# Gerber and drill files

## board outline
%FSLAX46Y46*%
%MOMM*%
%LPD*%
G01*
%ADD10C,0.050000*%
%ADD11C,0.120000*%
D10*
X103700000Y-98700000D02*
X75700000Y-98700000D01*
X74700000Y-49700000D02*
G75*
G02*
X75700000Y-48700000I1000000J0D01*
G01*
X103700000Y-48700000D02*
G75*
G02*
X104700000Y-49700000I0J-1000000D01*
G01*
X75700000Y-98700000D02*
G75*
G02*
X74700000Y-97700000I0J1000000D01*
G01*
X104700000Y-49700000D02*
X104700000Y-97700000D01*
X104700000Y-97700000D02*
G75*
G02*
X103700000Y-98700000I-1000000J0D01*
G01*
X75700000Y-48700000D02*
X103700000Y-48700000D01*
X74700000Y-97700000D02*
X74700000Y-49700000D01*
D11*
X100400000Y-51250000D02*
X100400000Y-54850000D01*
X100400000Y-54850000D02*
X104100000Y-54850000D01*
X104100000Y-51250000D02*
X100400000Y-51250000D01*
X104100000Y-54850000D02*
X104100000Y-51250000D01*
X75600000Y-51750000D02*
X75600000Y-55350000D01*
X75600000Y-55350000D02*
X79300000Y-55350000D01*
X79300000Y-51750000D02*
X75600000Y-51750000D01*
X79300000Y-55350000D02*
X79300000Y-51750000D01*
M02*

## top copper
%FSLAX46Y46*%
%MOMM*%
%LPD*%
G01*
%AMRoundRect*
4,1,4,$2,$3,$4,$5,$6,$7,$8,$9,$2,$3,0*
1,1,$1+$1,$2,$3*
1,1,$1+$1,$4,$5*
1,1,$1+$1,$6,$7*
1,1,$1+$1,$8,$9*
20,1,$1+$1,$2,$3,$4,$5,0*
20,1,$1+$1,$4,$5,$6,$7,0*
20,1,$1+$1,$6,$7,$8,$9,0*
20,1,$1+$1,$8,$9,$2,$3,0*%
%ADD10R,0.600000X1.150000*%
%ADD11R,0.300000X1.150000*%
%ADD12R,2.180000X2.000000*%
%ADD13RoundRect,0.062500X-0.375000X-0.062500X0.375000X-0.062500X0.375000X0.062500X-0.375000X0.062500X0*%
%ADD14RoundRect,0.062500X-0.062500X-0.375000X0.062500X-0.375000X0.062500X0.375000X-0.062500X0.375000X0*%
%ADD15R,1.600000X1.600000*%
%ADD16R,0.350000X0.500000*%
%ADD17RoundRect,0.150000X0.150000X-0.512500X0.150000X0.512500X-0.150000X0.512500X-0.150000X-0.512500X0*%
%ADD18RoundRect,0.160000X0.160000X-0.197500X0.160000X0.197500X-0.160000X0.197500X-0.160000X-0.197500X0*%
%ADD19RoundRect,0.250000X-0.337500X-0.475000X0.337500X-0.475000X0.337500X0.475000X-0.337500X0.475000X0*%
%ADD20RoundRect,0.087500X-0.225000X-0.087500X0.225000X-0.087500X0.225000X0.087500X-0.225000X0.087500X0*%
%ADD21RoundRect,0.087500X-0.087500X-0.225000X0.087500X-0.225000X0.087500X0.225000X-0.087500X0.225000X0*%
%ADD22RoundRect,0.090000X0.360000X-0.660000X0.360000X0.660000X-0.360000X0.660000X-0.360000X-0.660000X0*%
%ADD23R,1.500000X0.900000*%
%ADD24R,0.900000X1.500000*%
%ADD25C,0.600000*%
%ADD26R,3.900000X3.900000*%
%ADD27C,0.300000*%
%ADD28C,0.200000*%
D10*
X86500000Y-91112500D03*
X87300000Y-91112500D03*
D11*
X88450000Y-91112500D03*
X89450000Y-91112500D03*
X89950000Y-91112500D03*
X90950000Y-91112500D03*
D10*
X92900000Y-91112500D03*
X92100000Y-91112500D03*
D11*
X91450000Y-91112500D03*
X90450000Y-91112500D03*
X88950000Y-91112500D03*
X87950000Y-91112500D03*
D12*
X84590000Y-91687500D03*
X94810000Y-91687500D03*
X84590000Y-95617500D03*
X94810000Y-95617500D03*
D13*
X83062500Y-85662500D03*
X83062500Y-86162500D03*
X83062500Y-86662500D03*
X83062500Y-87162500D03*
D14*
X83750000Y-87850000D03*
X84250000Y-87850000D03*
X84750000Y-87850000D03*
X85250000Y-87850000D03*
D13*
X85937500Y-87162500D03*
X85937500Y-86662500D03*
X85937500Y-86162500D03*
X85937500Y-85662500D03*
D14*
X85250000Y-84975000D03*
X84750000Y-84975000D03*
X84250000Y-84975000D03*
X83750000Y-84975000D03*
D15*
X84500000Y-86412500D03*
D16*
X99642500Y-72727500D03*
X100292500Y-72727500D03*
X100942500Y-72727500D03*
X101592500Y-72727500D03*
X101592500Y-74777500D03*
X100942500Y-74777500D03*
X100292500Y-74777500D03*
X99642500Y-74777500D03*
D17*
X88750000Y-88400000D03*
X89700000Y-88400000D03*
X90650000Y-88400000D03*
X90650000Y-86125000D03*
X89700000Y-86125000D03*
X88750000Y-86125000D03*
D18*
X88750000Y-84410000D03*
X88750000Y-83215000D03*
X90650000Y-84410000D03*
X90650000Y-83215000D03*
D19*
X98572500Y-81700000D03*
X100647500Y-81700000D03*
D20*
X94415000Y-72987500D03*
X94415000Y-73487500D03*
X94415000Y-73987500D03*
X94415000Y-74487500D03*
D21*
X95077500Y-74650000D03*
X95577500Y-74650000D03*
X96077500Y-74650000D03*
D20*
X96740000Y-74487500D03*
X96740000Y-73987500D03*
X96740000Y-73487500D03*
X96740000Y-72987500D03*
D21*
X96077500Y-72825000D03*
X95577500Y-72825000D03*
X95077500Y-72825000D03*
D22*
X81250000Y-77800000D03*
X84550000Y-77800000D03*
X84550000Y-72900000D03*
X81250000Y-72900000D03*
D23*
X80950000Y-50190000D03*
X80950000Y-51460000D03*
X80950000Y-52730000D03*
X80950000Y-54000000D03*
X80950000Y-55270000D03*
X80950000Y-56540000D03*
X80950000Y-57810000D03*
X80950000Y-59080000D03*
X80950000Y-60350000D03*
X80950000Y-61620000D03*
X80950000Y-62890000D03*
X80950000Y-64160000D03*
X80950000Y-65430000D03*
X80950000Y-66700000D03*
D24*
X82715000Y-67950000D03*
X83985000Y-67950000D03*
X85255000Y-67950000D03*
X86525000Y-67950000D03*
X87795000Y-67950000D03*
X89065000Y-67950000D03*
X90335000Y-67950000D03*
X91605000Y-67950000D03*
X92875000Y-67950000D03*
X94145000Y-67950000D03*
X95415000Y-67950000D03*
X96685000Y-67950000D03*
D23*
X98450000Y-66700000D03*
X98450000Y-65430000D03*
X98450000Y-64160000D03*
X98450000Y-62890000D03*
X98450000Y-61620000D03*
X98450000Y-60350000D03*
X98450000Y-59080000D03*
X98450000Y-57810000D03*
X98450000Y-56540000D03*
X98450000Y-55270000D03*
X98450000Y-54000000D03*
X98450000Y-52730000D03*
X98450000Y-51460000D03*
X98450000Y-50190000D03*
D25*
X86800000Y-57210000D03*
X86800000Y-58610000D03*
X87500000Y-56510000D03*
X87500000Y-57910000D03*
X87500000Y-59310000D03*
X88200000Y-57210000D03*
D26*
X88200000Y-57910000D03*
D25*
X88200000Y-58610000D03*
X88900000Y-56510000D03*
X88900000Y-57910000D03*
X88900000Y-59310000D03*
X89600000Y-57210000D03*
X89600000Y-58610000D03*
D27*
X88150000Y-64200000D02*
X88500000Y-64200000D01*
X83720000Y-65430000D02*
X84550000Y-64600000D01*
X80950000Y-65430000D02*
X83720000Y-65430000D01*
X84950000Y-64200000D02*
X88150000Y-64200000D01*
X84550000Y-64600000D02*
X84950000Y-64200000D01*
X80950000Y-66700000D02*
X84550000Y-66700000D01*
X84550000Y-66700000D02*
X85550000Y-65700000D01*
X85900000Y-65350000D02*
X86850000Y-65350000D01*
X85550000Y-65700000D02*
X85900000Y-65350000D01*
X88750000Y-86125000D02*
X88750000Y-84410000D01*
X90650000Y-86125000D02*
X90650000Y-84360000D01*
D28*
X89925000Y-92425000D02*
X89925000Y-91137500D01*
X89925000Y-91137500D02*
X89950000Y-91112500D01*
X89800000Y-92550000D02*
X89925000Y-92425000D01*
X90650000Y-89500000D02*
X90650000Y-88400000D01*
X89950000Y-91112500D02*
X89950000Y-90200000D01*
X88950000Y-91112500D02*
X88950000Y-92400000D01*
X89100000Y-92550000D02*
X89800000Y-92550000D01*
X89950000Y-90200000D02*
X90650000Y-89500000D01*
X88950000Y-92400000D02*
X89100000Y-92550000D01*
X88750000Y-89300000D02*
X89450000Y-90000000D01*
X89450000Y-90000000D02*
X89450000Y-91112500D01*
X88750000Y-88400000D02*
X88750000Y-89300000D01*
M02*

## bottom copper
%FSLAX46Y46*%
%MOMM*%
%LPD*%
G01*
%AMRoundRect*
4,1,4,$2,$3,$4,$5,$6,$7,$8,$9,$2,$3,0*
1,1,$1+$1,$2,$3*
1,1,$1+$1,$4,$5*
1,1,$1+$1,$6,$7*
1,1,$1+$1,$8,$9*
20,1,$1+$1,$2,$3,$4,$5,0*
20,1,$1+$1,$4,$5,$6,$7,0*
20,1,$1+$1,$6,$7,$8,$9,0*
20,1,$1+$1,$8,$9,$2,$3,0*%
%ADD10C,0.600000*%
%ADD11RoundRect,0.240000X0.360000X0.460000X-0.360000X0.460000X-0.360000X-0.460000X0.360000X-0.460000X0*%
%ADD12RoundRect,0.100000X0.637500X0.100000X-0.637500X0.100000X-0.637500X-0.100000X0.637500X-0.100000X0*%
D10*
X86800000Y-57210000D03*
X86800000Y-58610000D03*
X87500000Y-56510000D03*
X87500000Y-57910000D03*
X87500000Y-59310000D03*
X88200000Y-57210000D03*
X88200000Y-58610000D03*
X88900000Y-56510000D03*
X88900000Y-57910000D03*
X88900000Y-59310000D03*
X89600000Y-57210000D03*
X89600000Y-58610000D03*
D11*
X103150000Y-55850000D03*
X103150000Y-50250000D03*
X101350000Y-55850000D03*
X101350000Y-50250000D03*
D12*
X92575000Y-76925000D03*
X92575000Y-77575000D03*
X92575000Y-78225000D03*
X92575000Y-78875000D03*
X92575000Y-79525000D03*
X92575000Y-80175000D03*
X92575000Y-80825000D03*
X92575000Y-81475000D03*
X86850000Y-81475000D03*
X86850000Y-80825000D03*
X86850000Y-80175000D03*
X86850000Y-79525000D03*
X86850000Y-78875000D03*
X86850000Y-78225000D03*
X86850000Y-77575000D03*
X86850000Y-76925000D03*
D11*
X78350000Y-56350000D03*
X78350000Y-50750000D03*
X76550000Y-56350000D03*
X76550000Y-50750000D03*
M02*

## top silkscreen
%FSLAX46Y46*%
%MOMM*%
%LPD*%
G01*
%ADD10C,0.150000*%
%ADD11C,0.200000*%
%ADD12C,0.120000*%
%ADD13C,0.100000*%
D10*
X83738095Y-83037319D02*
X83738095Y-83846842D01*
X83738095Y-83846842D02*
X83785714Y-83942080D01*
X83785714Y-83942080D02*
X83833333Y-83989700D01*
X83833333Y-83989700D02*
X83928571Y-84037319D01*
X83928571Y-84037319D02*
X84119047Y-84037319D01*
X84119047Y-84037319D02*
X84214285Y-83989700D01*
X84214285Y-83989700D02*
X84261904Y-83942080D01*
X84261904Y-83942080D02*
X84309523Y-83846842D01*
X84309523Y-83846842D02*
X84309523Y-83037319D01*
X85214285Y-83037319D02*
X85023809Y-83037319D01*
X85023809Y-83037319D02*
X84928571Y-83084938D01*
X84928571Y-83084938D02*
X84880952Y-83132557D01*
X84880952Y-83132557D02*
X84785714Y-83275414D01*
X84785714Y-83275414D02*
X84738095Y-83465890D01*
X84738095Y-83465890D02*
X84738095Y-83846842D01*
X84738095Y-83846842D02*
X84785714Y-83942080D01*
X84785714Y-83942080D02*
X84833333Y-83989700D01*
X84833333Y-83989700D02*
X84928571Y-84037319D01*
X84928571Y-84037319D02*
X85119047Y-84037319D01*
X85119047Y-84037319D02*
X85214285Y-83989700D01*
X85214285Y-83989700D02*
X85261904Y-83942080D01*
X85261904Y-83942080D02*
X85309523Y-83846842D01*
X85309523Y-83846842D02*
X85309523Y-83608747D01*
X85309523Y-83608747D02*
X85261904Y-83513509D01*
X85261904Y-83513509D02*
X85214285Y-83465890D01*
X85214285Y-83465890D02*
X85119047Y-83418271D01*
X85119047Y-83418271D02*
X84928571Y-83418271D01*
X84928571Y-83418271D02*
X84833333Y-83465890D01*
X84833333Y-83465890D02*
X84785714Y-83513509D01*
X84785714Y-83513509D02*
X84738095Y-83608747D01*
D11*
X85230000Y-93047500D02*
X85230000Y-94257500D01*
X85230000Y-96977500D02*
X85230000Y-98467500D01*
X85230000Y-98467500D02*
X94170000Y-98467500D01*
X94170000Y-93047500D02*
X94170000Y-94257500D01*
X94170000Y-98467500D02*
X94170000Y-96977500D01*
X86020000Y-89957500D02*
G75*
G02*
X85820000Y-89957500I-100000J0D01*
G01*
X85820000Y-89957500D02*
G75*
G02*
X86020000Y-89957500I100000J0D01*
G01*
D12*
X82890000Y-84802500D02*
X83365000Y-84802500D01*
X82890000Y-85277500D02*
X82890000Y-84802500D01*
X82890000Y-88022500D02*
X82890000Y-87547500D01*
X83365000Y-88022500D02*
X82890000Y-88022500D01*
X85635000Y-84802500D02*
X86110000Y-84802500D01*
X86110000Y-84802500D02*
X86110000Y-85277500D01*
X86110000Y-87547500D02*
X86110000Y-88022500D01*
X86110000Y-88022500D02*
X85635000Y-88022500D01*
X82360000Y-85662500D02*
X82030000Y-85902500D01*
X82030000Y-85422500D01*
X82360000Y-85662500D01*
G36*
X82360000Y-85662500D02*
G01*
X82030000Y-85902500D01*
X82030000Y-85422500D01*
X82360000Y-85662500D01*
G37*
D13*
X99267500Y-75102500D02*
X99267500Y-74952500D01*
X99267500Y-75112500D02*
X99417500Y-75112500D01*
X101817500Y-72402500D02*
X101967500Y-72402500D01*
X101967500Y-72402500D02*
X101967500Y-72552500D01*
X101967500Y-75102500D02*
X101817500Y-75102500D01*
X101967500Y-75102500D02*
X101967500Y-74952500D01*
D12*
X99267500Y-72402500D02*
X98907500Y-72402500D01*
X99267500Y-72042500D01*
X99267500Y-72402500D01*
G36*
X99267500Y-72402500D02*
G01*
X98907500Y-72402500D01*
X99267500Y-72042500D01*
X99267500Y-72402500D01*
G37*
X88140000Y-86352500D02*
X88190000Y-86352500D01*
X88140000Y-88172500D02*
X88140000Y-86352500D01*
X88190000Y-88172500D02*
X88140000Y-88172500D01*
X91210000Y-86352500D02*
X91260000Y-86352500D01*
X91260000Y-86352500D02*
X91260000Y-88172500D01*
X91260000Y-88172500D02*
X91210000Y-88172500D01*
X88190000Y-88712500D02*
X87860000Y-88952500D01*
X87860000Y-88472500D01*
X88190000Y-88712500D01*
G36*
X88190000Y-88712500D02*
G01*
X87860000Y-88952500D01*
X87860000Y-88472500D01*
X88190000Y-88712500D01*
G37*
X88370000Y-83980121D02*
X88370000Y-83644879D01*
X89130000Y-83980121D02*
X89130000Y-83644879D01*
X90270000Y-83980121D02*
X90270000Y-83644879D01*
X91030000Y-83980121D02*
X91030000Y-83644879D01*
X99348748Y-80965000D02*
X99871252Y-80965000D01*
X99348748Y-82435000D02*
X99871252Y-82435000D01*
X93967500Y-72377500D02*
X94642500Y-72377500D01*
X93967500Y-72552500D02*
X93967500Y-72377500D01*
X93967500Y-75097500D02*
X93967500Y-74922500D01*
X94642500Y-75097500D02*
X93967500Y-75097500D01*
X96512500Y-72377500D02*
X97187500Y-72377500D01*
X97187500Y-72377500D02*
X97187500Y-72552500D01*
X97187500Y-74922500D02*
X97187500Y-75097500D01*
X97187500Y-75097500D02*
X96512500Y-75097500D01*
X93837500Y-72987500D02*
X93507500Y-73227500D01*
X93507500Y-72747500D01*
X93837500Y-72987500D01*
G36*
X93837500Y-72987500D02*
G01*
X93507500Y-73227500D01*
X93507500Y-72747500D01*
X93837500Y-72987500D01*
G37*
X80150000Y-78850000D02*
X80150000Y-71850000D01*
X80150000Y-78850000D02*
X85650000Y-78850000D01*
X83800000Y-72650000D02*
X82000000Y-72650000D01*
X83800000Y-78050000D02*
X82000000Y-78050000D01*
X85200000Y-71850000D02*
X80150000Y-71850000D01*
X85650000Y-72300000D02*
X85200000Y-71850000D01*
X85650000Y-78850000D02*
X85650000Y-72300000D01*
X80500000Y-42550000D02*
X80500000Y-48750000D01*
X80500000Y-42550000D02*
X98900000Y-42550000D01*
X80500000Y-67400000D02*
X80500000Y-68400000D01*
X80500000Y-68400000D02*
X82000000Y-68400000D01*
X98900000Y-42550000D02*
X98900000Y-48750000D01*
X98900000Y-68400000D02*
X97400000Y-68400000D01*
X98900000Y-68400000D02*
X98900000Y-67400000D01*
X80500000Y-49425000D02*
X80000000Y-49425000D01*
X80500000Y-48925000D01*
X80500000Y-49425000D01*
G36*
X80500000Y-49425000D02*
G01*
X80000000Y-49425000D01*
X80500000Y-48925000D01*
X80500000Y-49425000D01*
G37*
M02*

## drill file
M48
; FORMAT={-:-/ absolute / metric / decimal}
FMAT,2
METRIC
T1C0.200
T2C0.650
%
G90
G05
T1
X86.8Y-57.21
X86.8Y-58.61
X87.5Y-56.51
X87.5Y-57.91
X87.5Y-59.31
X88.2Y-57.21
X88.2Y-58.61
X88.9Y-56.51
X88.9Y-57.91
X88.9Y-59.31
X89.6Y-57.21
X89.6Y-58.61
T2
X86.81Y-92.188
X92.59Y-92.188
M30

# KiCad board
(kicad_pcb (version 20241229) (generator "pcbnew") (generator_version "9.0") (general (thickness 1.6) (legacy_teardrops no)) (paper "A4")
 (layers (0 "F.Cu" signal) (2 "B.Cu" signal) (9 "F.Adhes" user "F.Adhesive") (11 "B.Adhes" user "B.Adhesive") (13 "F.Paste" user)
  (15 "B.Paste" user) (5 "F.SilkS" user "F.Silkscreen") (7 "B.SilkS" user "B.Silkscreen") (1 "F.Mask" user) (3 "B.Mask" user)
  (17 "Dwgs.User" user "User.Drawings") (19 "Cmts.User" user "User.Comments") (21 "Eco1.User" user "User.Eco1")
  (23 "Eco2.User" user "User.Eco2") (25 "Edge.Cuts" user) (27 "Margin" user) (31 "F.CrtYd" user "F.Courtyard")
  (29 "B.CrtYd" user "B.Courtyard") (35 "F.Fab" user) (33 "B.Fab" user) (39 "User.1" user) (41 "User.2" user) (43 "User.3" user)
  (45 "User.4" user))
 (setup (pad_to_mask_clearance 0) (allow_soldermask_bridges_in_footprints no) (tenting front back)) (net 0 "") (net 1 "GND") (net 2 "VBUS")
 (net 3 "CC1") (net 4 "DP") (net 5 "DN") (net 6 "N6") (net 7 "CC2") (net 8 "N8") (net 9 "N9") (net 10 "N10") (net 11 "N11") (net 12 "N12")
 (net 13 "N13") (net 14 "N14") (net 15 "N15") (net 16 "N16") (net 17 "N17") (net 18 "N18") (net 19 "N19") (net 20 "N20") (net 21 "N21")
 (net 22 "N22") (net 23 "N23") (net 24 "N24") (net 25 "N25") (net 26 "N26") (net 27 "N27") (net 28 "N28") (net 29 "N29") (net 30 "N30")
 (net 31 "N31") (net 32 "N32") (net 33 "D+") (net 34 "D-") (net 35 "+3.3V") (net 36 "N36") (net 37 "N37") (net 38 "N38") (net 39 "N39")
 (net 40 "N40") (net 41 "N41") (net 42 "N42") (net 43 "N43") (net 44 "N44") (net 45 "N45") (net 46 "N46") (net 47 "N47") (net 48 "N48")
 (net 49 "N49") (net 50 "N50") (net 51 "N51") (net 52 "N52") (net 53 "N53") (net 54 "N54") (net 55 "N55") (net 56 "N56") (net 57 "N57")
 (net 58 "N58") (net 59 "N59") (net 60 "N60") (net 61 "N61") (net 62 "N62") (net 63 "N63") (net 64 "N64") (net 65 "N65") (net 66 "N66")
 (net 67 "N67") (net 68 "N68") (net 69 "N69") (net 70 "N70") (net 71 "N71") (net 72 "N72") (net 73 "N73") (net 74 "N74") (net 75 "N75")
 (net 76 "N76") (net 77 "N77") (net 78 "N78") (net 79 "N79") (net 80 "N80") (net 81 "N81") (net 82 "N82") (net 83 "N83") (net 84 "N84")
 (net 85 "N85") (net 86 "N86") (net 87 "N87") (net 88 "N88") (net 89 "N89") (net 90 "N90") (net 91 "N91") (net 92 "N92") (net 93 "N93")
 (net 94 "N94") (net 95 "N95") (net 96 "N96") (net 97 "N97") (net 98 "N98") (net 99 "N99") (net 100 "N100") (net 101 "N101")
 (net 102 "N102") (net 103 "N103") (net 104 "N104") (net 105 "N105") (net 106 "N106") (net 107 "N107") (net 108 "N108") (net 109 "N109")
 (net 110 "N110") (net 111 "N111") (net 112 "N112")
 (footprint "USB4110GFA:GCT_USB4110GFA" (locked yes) (layer "F.Cu") (at 89.7 92.1875)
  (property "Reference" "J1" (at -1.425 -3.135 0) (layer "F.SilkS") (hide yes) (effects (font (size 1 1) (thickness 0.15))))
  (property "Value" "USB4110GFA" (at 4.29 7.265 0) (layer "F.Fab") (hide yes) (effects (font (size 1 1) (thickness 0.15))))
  (fp_line (start -4.47 0.86) (end -4.47 2.07) (stroke (width 0.2) (type solid)) (layer "F.SilkS"))
  (fp_line (start -4.47 4.79) (end -4.47 6.28) (stroke (width 0.2) (type solid)) (layer "F.SilkS"))
  (fp_line (start -4.47 6.28) (end 4.47 6.28) (stroke (width 0.2) (type solid)) (layer "F.SilkS"))
  (fp_line (start 4.47 0.86) (end 4.47 2.07) (stroke (width 0.2) (type solid)) (layer "F.SilkS"))
  (fp_line (start 4.47 6.28) (end 4.47 4.79) (stroke (width 0.2) (type solid)) (layer "F.SilkS"))
  (fp_circle (center -3.78 -2.23) (end -3.68 -2.23) (stroke (width 0.2) (type solid)) (fill no) (layer "F.SilkS"))
  (pad "" np_thru_hole circle (at -2.89 0) (size 0.65 0.65) (drill 0.65) (layers "*.Cu" "*.Mask"))
  (pad "" np_thru_hole circle (at 2.89 0) (size 0.65 0.65) (drill 0.65) (layers "*.Cu" "*.Mask"))
  (pad "A1/B12" smd rect (at -3.2 -1.075) (size 0.6 1.15) (layers "F.Cu" "F.Mask" "F.Paste") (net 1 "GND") (solder_mask_margin 0.102))
  (pad "A4/B9" smd rect (at -2.4 -1.075) (size 0.6 1.15) (layers "F.Cu" "F.Mask" "F.Paste") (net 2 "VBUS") (solder_mask_margin 0.102))
  (pad "A5" smd rect (at -1.25 -1.075) (size 0.3 1.15) (layers "F.Cu" "F.Mask" "F.Paste") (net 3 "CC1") (solder_mask_margin 0.102))
  (pad "A6" smd rect (at -0.25 -1.075) (size 0.3 1.15) (layers "F.Cu" "F.Mask" "F.Paste") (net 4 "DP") (solder_mask_margin 0.102))
  (pad "A7" smd rect (at 0.25 -1.075) (size 0.3 1.15) (layers "F.Cu" "F.Mask" "F.Paste") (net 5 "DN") (solder_mask_margin 0.102))
  (pad "A8" smd rect (at 1.25 -1.075) (size 0.3 1.15) (layers "F.Cu" "F.Mask" "F.Paste") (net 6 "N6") (solder_mask_margin 0.102))
  (pad "B1/A12" smd rect (at 3.2 -1.075) (size 0.6 1.15) (layers "F.Cu" "F.Mask" "F.Paste") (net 1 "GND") (solder_mask_margin 0.102))
  (pad "B4/A9" smd rect (at 2.4 -1.075) (size 0.6 1.15) (layers "F.Cu" "F.Mask" "F.Paste") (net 2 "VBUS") (solder_mask_margin 0.102))
  (pad "B5" smd rect (at 1.75 -1.075) (size 0.3 1.15) (layers "F.Cu" "F.Mask" "F.Paste") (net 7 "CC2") (solder_mask_margin 0.102))
  (pad "B6" smd rect (at 0.75 -1.075) (size 0.3 1.15) (layers "F.Cu" "F.Mask" "F.Paste") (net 4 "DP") (solder_mask_margin 0.102))
  (pad "B7" smd rect (at -0.75 -1.075) (size 0.3 1.15) (layers "F.Cu" "F.Mask" "F.Paste") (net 5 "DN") (solder_mask_margin 0.102))
  (pad "B8" smd rect (at -1.75 -1.075) (size 0.3 1.15) (layers "F.Cu" "F.Mask" "F.Paste") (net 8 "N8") (solder_mask_margin 0.102))
  (pad "S1" smd rect (at -5.11 -0.5) (size 2.18 2) (layers "F.Cu" "F.Mask" "F.Paste") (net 1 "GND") (solder_mask_margin 0.102))
  (pad "S2" smd rect (at 5.11 -0.5) (size 2.18 2) (layers "F.Cu" "F.Mask" "F.Paste") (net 1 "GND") (solder_mask_margin 0.102))
  (pad "S3" smd rect (at -5.11 3.43) (size 2.18 2) (layers "F.Cu" "F.Mask" "F.Paste") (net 1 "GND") (solder_mask_margin 0.102))
  (pad "S4" smd rect (at 5.11 3.43) (size 2.18 2) (layers "F.Cu" "F.Mask" "F.Paste") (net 1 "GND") (solder_mask_margin 0.102)))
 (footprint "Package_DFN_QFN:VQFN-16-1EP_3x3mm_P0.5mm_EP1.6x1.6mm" (layer "F.Cu") (at 84.5 86.4125)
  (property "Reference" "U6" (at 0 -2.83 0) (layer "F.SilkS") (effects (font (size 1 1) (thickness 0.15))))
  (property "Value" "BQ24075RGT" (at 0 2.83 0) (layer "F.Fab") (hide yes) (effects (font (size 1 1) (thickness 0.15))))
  (fp_line (start -1.61 -1.61) (end -1.135 -1.61) (stroke (width 0.12) (type solid)) (layer "F.SilkS"))
  (fp_line (start -1.61 -1.135) (end -1.61 -1.61) (stroke (width 0.12) (type solid)) (layer "F.SilkS"))
  (fp_line (start -1.61 1.61) (end -1.61 1.135) (stroke (width 0.12) (type solid)) (layer "F.SilkS"))
  (fp_line (start -1.135 1.61) (end -1.61 1.61) (stroke (width 0.12) (type solid)) (layer "F.SilkS"))
  (fp_line (start 1.135 -1.61) (end 1.61 -1.61) (stroke (width 0.12) (type solid)) (layer "F.SilkS"))
  (fp_line (start 1.61 -1.61) (end 1.61 -1.135) (stroke (width 0.12) (type solid)) (layer "F.SilkS"))
  (fp_line (start 1.61 1.135) (end 1.61 1.61) (stroke (width 0.12) (type solid)) (layer "F.SilkS"))
  (fp_line (start 1.61 1.61) (end 1.135 1.61) (stroke (width 0.12) (type solid)) (layer "F.SilkS"))
  (fp_poly (pts (xy -2.14 -0.75) (xy -2.47 -0.51) (xy -2.47 -0.99)) (stroke (width 0.12) (type solid)) (fill yes) (layer "F.SilkS"))
  (pad "" smd roundrect (at -0.4 -0.4) (size 0.64 0.64) (layers "F.Paste") (roundrect_rratio 0.25))
  (pad "" smd roundrect (at -0.4 0.4) (size 0.64 0.64) (layers "F.Paste") (roundrect_rratio 0.25))
  (pad "" smd roundrect (at 0.4 -0.4) (size 0.64 0.64) (layers "F.Paste") (roundrect_rratio 0.25))
  (pad "" smd roundrect (at 0.4 0.4) (size 0.64 0.64) (layers "F.Paste") (roundrect_rratio 0.25))
  (pad "1" smd roundrect (at -1.4375 -0.75) (size 0.875 0.25) (layers "F.Cu" "F.Mask" "F.Paste") (roundrect_rratio 0.25) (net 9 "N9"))
  (pad "2" smd roundrect (at -1.4375 -0.25) (size 0.875 0.25) (layers "F.Cu" "F.Mask" "F.Paste") (roundrect_rratio 0.25) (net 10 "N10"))
  (pad "3" smd roundrect (at -1.4375 0.25) (size 0.875 0.25) (layers "F.Cu" "F.Mask" "F.Paste") (roundrect_rratio 0.25) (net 10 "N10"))
  (pad "4" smd roundrect (at -1.4375 0.75) (size 0.875 0.25) (layers "F.Cu" "F.Mask" "F.Paste") (roundrect_rratio 0.25) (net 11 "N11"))
  (pad "5" smd roundrect (at -0.75 1.4375) (size 0.25 0.875) (layers "F.Cu" "F.Mask" "F.Paste") (roundrect_rratio 0.25) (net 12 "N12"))
  (pad "6" smd roundrect (at -0.25 1.4375) (size 0.25 0.875) (layers "F.Cu" "F.Mask" "F.Paste") (roundrect_rratio 0.25) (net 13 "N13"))
  (pad "7" smd roundrect (at 0.25 1.4375) (size 0.25 0.875) (layers "F.Cu" "F.Mask" "F.Paste") (roundrect_rratio 0.25) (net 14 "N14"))
  (pad "8" smd roundrect (at 0.75 1.4375) (size 0.25 0.875) (layers "F.Cu" "F.Mask" "F.Paste") (roundrect_rratio 0.25) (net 1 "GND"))
  (pad "9" smd roundrect (at 1.4375 0.75) (size 0.875 0.25) (layers "F.Cu" "F.Mask" "F.Paste") (roundrect_rratio 0.25) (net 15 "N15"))
  (pad "10" smd roundrect (at 1.4375 0.25) (size 0.875 0.25) (layers "F.Cu" "F.Mask" "F.Paste") (roundrect_rratio 0.25) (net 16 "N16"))
  (pad "11" smd roundrect (at 1.4375 -0.25) (size 0.875 0.25) (layers "F.Cu" "F.Mask" "F.Paste") (roundrect_rratio 0.25) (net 16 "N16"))
  (pad "12" smd roundrect (at 1.4375 -0.75) (size 0.875 0.25) (layers "F.Cu" "F.Mask" "F.Paste") (roundrect_rratio 0.25) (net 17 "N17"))
  (pad "13" smd roundrect (at 0.75 -1.4375) (size 0.25 0.875) (layers "F.Cu" "F.Mask" "F.Paste") (roundrect_rratio 0.25) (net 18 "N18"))
  (pad "14" smd roundrect (at 0.25 -1.4375) (size 0.25 0.875) (layers "F.Cu" "F.Mask" "F.Paste") (roundrect_rratio 0.25) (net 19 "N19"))
  (pad "15" smd roundrect (at -0.25 -1.4375) (size 0.25 0.875) (layers "F.Cu" "F.Mask" "F.Paste") (roundrect_rratio 0.25) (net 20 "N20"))
  (pad "16" smd roundrect (at -0.75 -1.4375) (size 0.25 0.875) (layers "F.Cu" "F.Mask" "F.Paste") (roundrect_rratio 0.25) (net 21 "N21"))
  (pad "17" smd rect (at 0 0) (size 1.6 1.6) (layers "F.Cu" "F.Mask") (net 1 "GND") (zone_connect 2)))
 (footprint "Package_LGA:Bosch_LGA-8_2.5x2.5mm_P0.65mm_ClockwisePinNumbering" (layer "F.Cu") (at 100.6175 73.7525)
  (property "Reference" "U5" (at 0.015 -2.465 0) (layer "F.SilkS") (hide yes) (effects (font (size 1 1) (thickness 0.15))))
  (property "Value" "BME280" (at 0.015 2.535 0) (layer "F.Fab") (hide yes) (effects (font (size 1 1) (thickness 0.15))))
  (fp_line (start -1.35 1.35) (end -1.35 1.2) (stroke (width 0.1) (type solid)) (layer "F.SilkS"))
  (fp_line (start -1.35 1.36) (end -1.2 1.36) (stroke (width 0.1) (type solid)) (layer "F.SilkS"))
  (fp_line (start 1.2 -1.35) (end 1.35 -1.35) (stroke (width 0.1) (type solid)) (layer "F.SilkS"))
  (fp_line (start 1.35 -1.35) (end 1.35 -1.2) (stroke (width 0.1) (type solid)) (layer "F.SilkS"))
  (fp_line (start 1.35 1.35) (end 1.2 1.35) (stroke (width 0.1) (type solid)) (layer "F.SilkS"))
  (fp_line (start 1.35 1.35) (end 1.35 1.2) (stroke (width 0.1) (type solid)) (layer "F.SilkS"))
  (fp_poly
   (pts (xy -1.35 -1.35) (xy -1.71 -1.35) (xy -1.35 -1.71) (xy -1.35 -1.35)) (stroke (width 0.12) (type solid)) (fill yes) (layer "F.SilkS"))
  (pad "1" smd rect (at -0.975 -1.025 90) (size 0.5 0.35) (layers "F.Cu" "F.Mask" "F.Paste") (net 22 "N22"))
  (pad "2" smd rect (at -0.325 -1.025 90) (size 0.5 0.35) (layers "F.Cu" "F.Mask" "F.Paste") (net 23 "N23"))
  (pad "3" smd rect (at 0.325 -1.025 90) (size 0.5 0.35) (layers "F.Cu" "F.Mask" "F.Paste") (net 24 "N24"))
  (pad "4" smd rect (at 0.975 -1.025 90) (size 0.5 0.35) (layers "F.Cu" "F.Mask" "F.Paste") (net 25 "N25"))
  (pad "5" smd rect (at 0.975 1.025 90) (size 0.5 0.35) (layers "F.Cu" "F.Mask" "F.Paste") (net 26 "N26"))
  (pad "6" smd rect (at 0.325 1.025 90) (size 0.5 0.35) (layers "F.Cu" "F.Mask" "F.Paste") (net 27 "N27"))
  (pad "7" smd rect (at -0.325 1.025 90) (size 0.5 0.35) (layers "F.Cu" "F.Mask" "F.Paste") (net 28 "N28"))
  (pad "8" smd rect (at -0.975 1.025 90) (size 0.5 0.35) (layers "F.Cu" "F.Mask" "F.Paste") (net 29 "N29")))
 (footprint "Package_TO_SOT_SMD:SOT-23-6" (layer "F.Cu") (at 89.7 87.2625 90)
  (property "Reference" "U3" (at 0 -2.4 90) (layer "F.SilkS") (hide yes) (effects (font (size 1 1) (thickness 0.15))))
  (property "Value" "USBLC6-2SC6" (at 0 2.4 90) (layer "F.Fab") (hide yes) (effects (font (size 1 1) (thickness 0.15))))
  (fp_line (start 0.91 -1.56) (end 0.91 -1.51) (stroke (width 0.12) (type solid)) (layer "F.SilkS"))
  (fp_line (start -0.91 -1.56) (end 0.91 -1.56) (stroke (width 0.12) (type solid)) (layer "F.SilkS"))
  (fp_line (start -0.91 -1.51) (end -0.91 -1.56) (stroke (width 0.12) (type solid)) (layer "F.SilkS"))
  (fp_line (start 0.91 1.51) (end 0.91 1.56) (stroke (width 0.12) (type solid)) (layer "F.SilkS"))
  (fp_line (start 0.91 1.56) (end -0.91 1.56) (stroke (width 0.12) (type solid)) (layer "F.SilkS"))
  (fp_line (start -0.91 1.56) (end -0.91 1.51) (stroke (width 0.12) (type solid)) (layer "F.SilkS"))
  (fp_poly (pts (xy -1.45 -1.51) (xy -1.69 -1.84) (xy -1.21 -1.84)) (stroke (width 0.12) (type solid)) (fill yes) (layer "F.SilkS"))
  (pad "1" smd roundrect (at -1.1375 -0.95 90) (size 1.325 0.6) (layers "F.Cu" "F.Mask" "F.Paste") (roundrect_rratio 0.25) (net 4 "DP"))
  (pad "2" smd roundrect (at -1.1375 0 90) (size 1.325 0.6) (layers "F.Cu" "F.Mask" "F.Paste") (roundrect_rratio 0.25) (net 1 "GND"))
  (pad "3" smd roundrect (at -1.1375 0.95 90) (size 1.325 0.6) (layers "F.Cu" "F.Mask" "F.Paste") (roundrect_rratio 0.25) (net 5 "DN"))
  (pad "4" smd roundrect (at 1.1375 0.95 90) (size 1.325 0.6) (layers "F.Cu" "F.Mask" "F.Paste") (roundrect_rratio 0.25) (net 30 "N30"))
  (pad "5" smd roundrect (at 1.1375 0 90) (size 1.325 0.6) (layers "F.Cu" "F.Mask" "F.Paste") (roundrect_rratio 0.25) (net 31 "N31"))
  (pad "6" smd roundrect (at 1.1375 -0.95 90) (size 1.325 0.6) (layers "F.Cu" "F.Mask" "F.Paste") (roundrect_rratio 0.25) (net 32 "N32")))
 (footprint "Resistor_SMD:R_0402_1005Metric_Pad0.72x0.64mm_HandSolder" (layer "F.Cu") (at 88.75 83.8125 90)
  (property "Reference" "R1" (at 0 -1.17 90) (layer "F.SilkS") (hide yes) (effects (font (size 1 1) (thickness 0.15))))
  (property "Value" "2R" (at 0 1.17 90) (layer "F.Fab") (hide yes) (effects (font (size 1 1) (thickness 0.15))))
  (fp_line (start -0.167621 -0.38) (end 0.167621 -0.38) (stroke (width 0.12) (type solid)) (layer "F.SilkS"))
  (fp_line (start -0.167621 0.38) (end 0.167621 0.38) (stroke (width 0.12) (type solid)) (layer "F.SilkS"))
  (pad "1" smd roundrect (at -0.5975 0 90) (size 0.715 0.64) (layers "F.Cu" "F.Mask" "F.Paste") (roundrect_rratio 0.25) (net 32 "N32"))
  (pad "2" smd roundrect (at 0.5975 0 90) (size 0.715 0.64) (layers "F.Cu" "F.Mask" "F.Paste") (roundrect_rratio 0.25) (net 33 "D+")))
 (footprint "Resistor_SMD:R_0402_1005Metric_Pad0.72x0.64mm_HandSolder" (layer "F.Cu") (at 90.65 83.8125 90)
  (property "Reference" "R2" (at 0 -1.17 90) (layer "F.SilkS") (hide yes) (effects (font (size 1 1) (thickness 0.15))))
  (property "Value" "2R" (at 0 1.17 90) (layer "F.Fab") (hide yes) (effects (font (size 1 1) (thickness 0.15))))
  (fp_line (start -0.167621 -0.38) (end 0.167621 -0.38) (stroke (width 0.12) (type solid)) (layer "F.SilkS"))
  (fp_line (start -0.167621 0.38) (end 0.167621 0.38) (stroke (width 0.12) (type solid)) (layer "F.SilkS"))
  (pad "1" smd roundrect (at -0.5975 0 90) (size 0.715 0.64) (layers "F.Cu" "F.Mask" "F.Paste") (roundrect_rratio 0.25) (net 30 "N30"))
  (pad "2" smd roundrect (at 0.5975 0 90) (size 0.715 0.64) (layers "F.Cu" "F.Mask" "F.Paste") (roundrect_rratio 0.25) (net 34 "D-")))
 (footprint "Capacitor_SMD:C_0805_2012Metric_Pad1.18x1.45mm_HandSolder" (layer "F.Cu") (at 99.61 81.7)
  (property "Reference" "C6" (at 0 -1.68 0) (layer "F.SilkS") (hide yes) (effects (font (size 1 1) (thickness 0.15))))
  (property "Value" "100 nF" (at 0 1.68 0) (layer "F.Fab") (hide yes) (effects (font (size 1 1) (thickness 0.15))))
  (fp_line (start -0.261252 -0.735) (end 0.261252 -0.735) (stroke (width 0.12) (type solid)) (layer "F.SilkS"))
  (fp_line (start -0.261252 0.735) (end 0.261252 0.735) (stroke (width 0.12) (type solid)) (layer "F.SilkS"))
  (pad "1" smd roundrect (at -1.0375 0) (size 1.175 1.45) (layers "F.Cu" "F.Mask" "F.Paste") (roundrect_rratio 0.212766) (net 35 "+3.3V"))
  (pad "2" smd roundrect (at 1.0375 0) (size 1.175 1.45) (layers "F.Cu" "F.Mask" "F.Paste") (roundrect_rratio 0.212766) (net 1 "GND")))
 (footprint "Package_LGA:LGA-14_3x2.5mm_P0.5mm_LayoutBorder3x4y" (layer "F.Cu") (at 95.5775 73.7375)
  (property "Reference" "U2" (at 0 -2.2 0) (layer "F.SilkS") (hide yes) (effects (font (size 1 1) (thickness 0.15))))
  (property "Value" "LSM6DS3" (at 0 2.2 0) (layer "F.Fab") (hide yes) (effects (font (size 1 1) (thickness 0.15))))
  (fp_line (start -1.61 -1.36) (end -0.935 -1.36) (stroke (width 0.12) (type solid)) (layer "F.SilkS"))
  (fp_line (start -1.61 -1.185) (end -1.61 -1.36) (stroke (width 0.12) (type solid)) (layer "F.SilkS"))
  (fp_line (start -1.61 1.36) (end -1.61 1.185) (stroke (width 0.12) (type solid)) (layer "F.SilkS"))
  (fp_line (start -0.935 1.36) (end -1.61 1.36) (stroke (width 0.12) (type solid)) (layer "F.SilkS"))
  (fp_line (start 0.935 -1.36) (end 1.61 -1.36) (stroke (width 0.12) (type solid)) (layer "F.SilkS"))
  (fp_line (start 1.61 -1.36) (end 1.61 -1.185) (stroke (width 0.12) (type solid)) (layer "F.SilkS"))
  (fp_line (start 1.61 1.185) (end 1.61 1.36) (stroke (width 0.12) (type solid)) (layer "F.SilkS"))
  (fp_line (start 1.61 1.36) (end 0.935 1.36) (stroke (width 0.12) (type solid)) (layer "F.SilkS"))
  (fp_poly (pts (xy -1.74 -0.75) (xy -2.07 -0.51) (xy -2.07 -0.99)) (stroke (width 0.12) (type solid)) (fill yes) (layer "F.SilkS"))
  (pad "1" smd roundrect (at -1.1625 -0.75) (size 0.625 0.35) (layers "F.Cu" "F.Mask" "F.Paste") (roundrect_rratio 0.25) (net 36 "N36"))
  (pad "2" smd roundrect (at -1.1625 -0.25) (size 0.625 0.35) (layers "F.Cu" "F.Mask" "F.Paste") (roundrect_rratio 0.25) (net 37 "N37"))
  (pad "3" smd roundrect (at -1.1625 0.25) (size 0.625 0.35) (layers "F.Cu" "F.Mask" "F.Paste") (roundrect_rratio 0.25) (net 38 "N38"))
  (pad "4" smd roundrect (at -1.1625 0.75) (size 0.625 0.35) (layers "F.Cu" "F.Mask" "F.Paste") (roundrect_rratio 0.25) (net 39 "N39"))
  (pad "5" smd roundrect (at -0.5 0.9125) (size 0.35 0.625) (layers "F.Cu" "F.Mask" "F.Paste") (roundrect_rratio 0.25) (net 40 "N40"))
  (pad "6" smd roundrect (at 0 0.9125) (size 0.35 0.625) (layers "F.Cu" "F.Mask" "F.Paste") (roundrect_rratio 0.25) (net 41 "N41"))
  (pad "7" smd roundrect (at 0.5 0.9125) (size 0.35 0.625) (layers "F.Cu" "F.Mask" "F.Paste") (roundrect_rratio 0.25) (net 41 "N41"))
  (pad "8" smd roundrect (at 1.1625 0.75) (size 0.625 0.35) (layers "F.Cu" "F.Mask" "F.Paste") (roundrect_rratio 0.25) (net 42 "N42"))
  (pad "9" smd roundrect (at 1.1625 0.25) (size 0.625 0.35) (layers "F.Cu" "F.Mask" "F.Paste") (roundrect_rratio 0.25) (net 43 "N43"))
  (pad "10" smd roundrect (at 1.1625 -0.25) (size 0.625 0.35) (layers "F.Cu" "F.Mask" "F.Paste") (roundrect_rratio 0.25) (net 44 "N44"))
  (pad "11" smd roundrect (at 1.1625 -0.75) (size 0.625 0.35) (layers "F.Cu" "F.Mask" "F.Paste") (roundrect_rratio 0.25) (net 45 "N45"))
  (pad "12" smd roundrect (at 0.5 -0.9125) (size 0.35 0.625) (layers "F.Cu" "F.Mask" "F.Paste") (roundrect_rratio 0.25) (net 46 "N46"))
  (pad "13" smd roundrect (at 0 -0.9125) (size 0.35 0.625) (layers "F.Cu" "F.Mask" "F.Paste") (roundrect_rratio 0.25) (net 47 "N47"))
  (pad "14" smd roundrect (at -0.5 -0.9125) (size 0.35 0.625) (layers "F.Cu" "F.Mask" "F.Paste") (roundrect_rratio 0.25) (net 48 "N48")))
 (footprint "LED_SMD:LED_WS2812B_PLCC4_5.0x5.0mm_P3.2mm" (layer "F.Cu") (at 82.9 75.35 90)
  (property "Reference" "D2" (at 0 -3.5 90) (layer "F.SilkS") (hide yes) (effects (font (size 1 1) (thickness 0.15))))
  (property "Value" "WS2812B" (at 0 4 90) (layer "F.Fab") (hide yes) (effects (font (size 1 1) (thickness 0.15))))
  (fp_line (start -3.5 -2.75) (end 3.5 -2.75) (stroke (width 0.12) (type solid)) (layer "F.SilkS"))
  (fp_line (start -3.5 -2.75) (end -3.5 2.75) (stroke (width 0.12) (type default)) (layer "F.SilkS"))
  (fp_line (start 2.7 0.9) (end 2.7 -0.9) (stroke (width 0.12) (type default)) (layer "F.SilkS"))
  (fp_line (start -2.7 0.9) (end -2.7 -0.9) (stroke (width 0.12) (type default)) (layer "F.SilkS"))
  (fp_line (start 3.5 2.3) (end 3.5 -2.75) (stroke (width 0.12) (type default)) (layer "F.SilkS"))
  (fp_line (start 3.05 2.75) (end 3.5 2.3) (stroke (width 0.12) (type default)) (layer "F.SilkS"))
  (fp_line (start -3.5 2.75) (end 3.05 2.75) (stroke (width 0.12) (type solid)) (layer "F.SilkS"))
  (pad "1" smd roundrect (at -2.45 -1.65 90) (size 1.5 0.9) (layers "F.Cu" "F.Mask" "F.Paste") (roundrect_rratio 0.1) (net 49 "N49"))
  (pad "2" smd roundrect (at -2.45 1.65 90) (size 1.5 0.9) (layers "F.Cu" "F.Mask" "F.Paste") (roundrect_rratio 0.1) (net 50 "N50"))
  (pad "3" smd roundrect (at 2.45 1.65 90) (size 1.5 0.9) (layers "F.Cu" "F.Mask" "F.Paste") (roundrect_rratio 0.1) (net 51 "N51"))
  (pad "4" smd roundrect (at 2.45 -1.65 90) (size 1.5 0.9) (layers "F.Cu" "F.Mask" "F.Paste") (roundrect_rratio 0.1) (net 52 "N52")))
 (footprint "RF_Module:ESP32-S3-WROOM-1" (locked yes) (layer "F.Cu") (at 89.7 55.45)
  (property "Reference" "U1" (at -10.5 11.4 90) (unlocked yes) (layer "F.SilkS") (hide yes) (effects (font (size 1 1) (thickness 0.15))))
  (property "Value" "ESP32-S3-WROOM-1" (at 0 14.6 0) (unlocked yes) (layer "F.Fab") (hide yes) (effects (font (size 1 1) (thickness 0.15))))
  (fp_line (start -9.2 -12.9) (end -9.2 -6.7) (stroke (width 0.12) (type solid)) (layer "F.SilkS"))
  (fp_line (start -9.2 -12.9) (end 9.2 -12.9) (stroke (width 0.12) (type solid)) (layer "F.SilkS"))
  (fp_line (start -9.2 11.95) (end -9.2 12.95) (stroke (width 0.12) (type solid)) (layer "F.SilkS"))
  (fp_line (start -9.2 12.95) (end -7.7 12.95) (stroke (width 0.12) (type solid)) (layer "F.SilkS"))
  (fp_line (start 9.2 -12.9) (end 9.2 -6.7) (stroke (width 0.12) (type solid)) (layer "F.SilkS"))
  (fp_line (start 9.2 12.95) (end 7.7 12.95) (stroke (width 0.12) (type solid)) (layer "F.SilkS"))
  (fp_line (start 9.2 12.95) (end 9.2 11.95) (stroke (width 0.12) (type solid)) (layer "F.SilkS"))
  (fp_poly
   (pts (xy -9.2 -6.025) (xy -9.7 -6.025) (xy -9.2 -6.525) (xy -9.2 -6.025)) (stroke (width 0.12) (type solid)) (fill yes) (layer "F.SilkS"))
  (pad "" smd rect (at -2.9 1.06) (size 0.9 0.9) (layers "F.Paste"))
  (pad "" smd rect (at -2.9 2.46 270) (size 0.9 0.9) (layers "F.Paste"))
  (pad "" smd rect (at -2.9 3.86) (size 0.9 0.9) (layers "F.Paste"))
  (pad "" smd rect (at -1.5 1.06 270) (size 0.9 0.9) (layers "F.Paste"))
  (pad "" smd rect (at -1.5 2.46 270) (size 0.9 0.9) (layers "F.Paste"))
  (pad "" smd rect (at -1.5 3.86 270) (size 0.9 0.9) (layers "F.Paste"))
  (pad "" smd rect (at -0.1 1.06 270) (size 0.9 0.9) (layers "F.Paste"))
  (pad "" smd rect (at -0.1 2.46 270) (size 0.9 0.9) (layers "F.Paste"))
  (pad "" smd rect (at -0.1 3.86 270) (size 0.9 0.9) (layers "F.Paste"))
  (pad "1" smd rect (at -8.75 -5.26) (size 1.5 0.9) (layers "F.Cu" "F.Mask" "F.Paste") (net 1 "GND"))
  (pad "2" smd rect (at -8.75 -3.99) (size 1.5 0.9) (layers "F.Cu" "F.Mask" "F.Paste") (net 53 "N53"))
  (pad "3" smd rect (at -8.75 -2.72) (size 1.5 0.9) (layers "F.Cu" "F.Mask" "F.Paste") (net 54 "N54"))
  (pad "4" smd rect (at -8.75 -1.45) (size 1.5 0.9) (layers "F.Cu" "F.Mask" "F.Paste") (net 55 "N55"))
  (pad "5" smd rect (at -8.75 -0.18) (size 1.5 0.9) (layers "F.Cu" "F.Mask" "F.Paste") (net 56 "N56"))
  (pad "6" smd rect (at -8.75 1.09) (size 1.5 0.9) (layers "F.Cu" "F.Mask" "F.Paste") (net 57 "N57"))
  (pad "7" smd rect (at -8.75 2.36) (size 1.5 0.9) (layers "F.Cu" "F.Mask" "F.Paste") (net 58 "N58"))
  (pad "8" smd rect (at -8.75 3.63) (size 1.5 0.9) (layers "F.Cu" "F.Mask" "F.Paste") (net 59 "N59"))
  (pad "9" smd rect (at -8.75 4.9) (size 1.5 0.9) (layers "F.Cu" "F.Mask" "F.Paste") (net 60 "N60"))
  (pad "10" smd rect (at -8.75 6.17) (size 1.5 0.9) (layers "F.Cu" "F.Mask" "F.Paste") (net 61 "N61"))
  (pad "11" smd rect (at -8.75 7.44) (size 1.5 0.9) (layers "F.Cu" "F.Mask" "F.Paste") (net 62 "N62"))
  (pad "12" smd rect (at -8.75 8.71) (size 1.5 0.9) (layers "F.Cu" "F.Mask" "F.Paste") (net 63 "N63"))
  (pad "13" smd rect (at -8.75 9.98) (size 1.5 0.9) (layers "F.Cu" "F.Mask" "F.Paste") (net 34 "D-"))
  (pad "14" smd rect (at -8.75 11.25 180) (size 1.5 0.9) (layers "F.Cu" "F.Mask" "F.Paste") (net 33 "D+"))
  (pad "15" smd rect (at -6.985 12.5 270) (size 1.5 0.9) (layers "F.Cu" "F.Mask" "F.Paste") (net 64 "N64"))
  (pad "16" smd rect (at -5.715 12.5 270) (size 1.5 0.9) (layers "F.Cu" "F.Mask" "F.Paste") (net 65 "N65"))
  (pad "17" smd rect (at -4.445 12.5 270) (size 1.5 0.9) (layers "F.Cu" "F.Mask" "F.Paste") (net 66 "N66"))
  (pad "18" smd rect (at -3.175 12.5 270) (size 1.5 0.9) (layers "F.Cu" "F.Mask" "F.Paste") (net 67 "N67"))
  (pad "19" smd rect (at -1.905 12.5 270) (size 1.5 0.9) (layers "F.Cu" "F.Mask" "F.Paste") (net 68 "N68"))
  (pad "20" smd rect (at -0.635 12.5 270) (size 1.5 0.9) (layers "F.Cu" "F.Mask" "F.Paste") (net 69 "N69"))
  (pad "21" smd rect (at 0.635 12.5 270) (size 1.5 0.9) (layers "F.Cu" "F.Mask" "F.Paste") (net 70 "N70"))
  (pad "22" smd rect (at 1.905 12.5 270) (size 1.5 0.9) (layers "F.Cu" "F.Mask" "F.Paste") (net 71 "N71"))
  (pad "23" smd rect (at 3.175 12.5 270) (size 1.5 0.9) (layers "F.Cu" "F.Mask" "F.Paste") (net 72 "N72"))
  (pad "24" smd rect (at 4.445 12.5 270) (size 1.5 0.9) (layers "F.Cu" "F.Mask" "F.Paste") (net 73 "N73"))
  (pad "25" smd rect (at 5.715 12.5 270) (size 1.5 0.9) (layers "F.Cu" "F.Mask" "F.Paste") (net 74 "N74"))
  (pad "26" smd rect (at 6.985 12.5 270) (size 1.5 0.9) (layers "F.Cu" "F.Mask" "F.Paste") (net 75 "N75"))
  (pad "27" smd rect (at 8.75 11.25) (size 1.5 0.9) (layers "F.Cu" "F.Mask" "F.Paste") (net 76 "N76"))
  (pad "28" smd rect (at 8.75 9.98) (size 1.5 0.9) (layers "F.Cu" "F.Mask" "F.Paste") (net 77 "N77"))
  (pad "29" smd rect (at 8.75 8.71) (size 1.5 0.9) (layers "F.Cu" "F.Mask" "F.Paste") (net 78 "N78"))
  (pad "30" smd rect (at 8.75 7.44) (size 1.5 0.9) (layers "F.Cu" "F.Mask" "F.Paste") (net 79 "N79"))
  (pad "31" smd rect (at 8.75 6.17) (size 1.5 0.9) (layers "F.Cu" "F.Mask" "F.Paste") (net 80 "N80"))
  (pad "32" smd rect (at 8.75 4.9) (size 1.5 0.9) (layers "F.Cu" "F.Mask" "F.Paste") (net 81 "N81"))
  (pad "33" smd rect (at 8.75 3.63) (size 1.5 0.9) (layers "F.Cu" "F.Mask" "F.Paste") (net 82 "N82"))
  (pad "34" smd rect (at 8.75 2.36) (size 1.5 0.9) (layers "F.Cu" "F.Mask" "F.Paste") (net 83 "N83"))
  (pad "35" smd rect (at 8.75 1.09) (size 1.5 0.9) (layers "F.Cu" "F.Mask" "F.Paste") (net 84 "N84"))
  (pad "36" smd rect (at 8.75 -0.18) (size 1.5 0.9) (layers "F.Cu" "F.Mask" "F.Paste") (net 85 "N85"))
  (pad "37" smd rect (at 8.75 -1.45) (size 1.5 0.9) (layers "F.Cu" "F.Mask" "F.Paste") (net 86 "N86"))
  (pad "38" smd rect (at 8.75 -2.72) (size 1.5 0.9) (layers "F.Cu" "F.Mask" "F.Paste") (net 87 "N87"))
  (pad "39" smd rect (at 8.75 -3.99) (size 1.5 0.9) (layers "F.Cu" "F.Mask" "F.Paste") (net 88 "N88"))
  (pad "40" smd rect (at 8.75 -5.26) (size 1.5 0.9) (layers "F.Cu" "F.Mask" "F.Paste") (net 1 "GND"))
  (pad "41" thru_hole circle (at -2.9 1.76 90) (size 0.6 0.6) (drill 0.2) (layers "*.Cu" "F.Mask") (remove_unused_layers no) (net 1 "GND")
   (zone_connect 2))
  (pad "41" thru_hole circle (at -2.9 3.16) (size 0.6 0.6) (drill 0.2) (layers "*.Cu" "F.Mask") (remove_unused_layers no) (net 1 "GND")
   (zone_connect 2))
  (pad "41" thru_hole circle (at -2.2 1.06) (size 0.6 0.6) (drill 0.2) (layers "*.Cu" "F.Mask") (remove_unused_layers no) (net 1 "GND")
   (zone_connect 2))
  (pad "41" thru_hole circle (at -2.2 2.46) (size 0.6 0.6) (drill 0.2) (layers "*.Cu" "F.Mask") (remove_unused_layers no) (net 1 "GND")
   (zone_connect 2))
  (pad "41" thru_hole circle (at -2.2 3.86) (size 0.6 0.6) (drill 0.2) (layers "*.Cu" "F.Mask") (remove_unused_layers no) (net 1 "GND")
   (zone_connect 2))
  (pad "41" thru_hole circle (at -1.5 1.76) (size 0.6 0.6) (drill 0.2) (layers "*.Cu" "F.Mask") (remove_unused_layers no) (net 1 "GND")
   (zone_connect 2))
  (pad "41" smd rect (at -1.5 2.46 270) (size 3.9 3.9) (layers "F.Cu" "F.Mask") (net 1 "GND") (zone_connect 2))
  (pad "41" thru_hole circle (at -1.5 3.16) (size 0.6 0.6) (drill 0.2) (layers "*.Cu" "F.Mask") (remove_unused_layers no) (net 1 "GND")
   (zone_connect 2))
  (pad "41" thru_hole circle (at -0.8 1.06) (size 0.6 0.6) (drill 0.2) (layers "*.Cu" "F.Mask") (remove_unused_layers no) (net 1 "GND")
   (zone_connect 2))
  (pad "41" thru_hole circle (at -0.8 2.46) (size 0.6 0.6) (drill 0.2) (layers "*.Cu" "F.Mask") (remove_unused_layers no) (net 1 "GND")
   (zone_connect 2))
  (pad "41" thru_hole circle (at -0.8 3.86) (size 0.6 0.6) (drill 0.2) (layers "*.Cu" "F.Mask") (remove_unused_layers no) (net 1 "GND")
   (zone_connect 2))
  (pad "41" thru_hole circle (at -0.1 1.76) (size 0.6 0.6) (drill 0.2) (layers "*.Cu" "F.Mask") (remove_unused_layers no) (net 1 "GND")
   (zone_connect 2))
  (pad "41" thru_hole circle (at -0.1 3.16) (size 0.6 0.6) (drill 0.2) (layers "*.Cu" "F.Mask") (remove_unused_layers no) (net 1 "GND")
   (zone_connect 2))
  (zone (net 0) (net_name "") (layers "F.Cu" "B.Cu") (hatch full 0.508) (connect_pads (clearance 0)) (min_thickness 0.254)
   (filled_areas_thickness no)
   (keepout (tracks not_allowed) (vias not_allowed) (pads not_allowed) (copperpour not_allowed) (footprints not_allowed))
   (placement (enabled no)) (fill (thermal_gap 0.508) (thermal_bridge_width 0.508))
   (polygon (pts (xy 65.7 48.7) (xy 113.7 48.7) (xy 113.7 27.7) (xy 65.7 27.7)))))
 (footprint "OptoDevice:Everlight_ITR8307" (layer "B.Cu") (at 102.25 53.05 180)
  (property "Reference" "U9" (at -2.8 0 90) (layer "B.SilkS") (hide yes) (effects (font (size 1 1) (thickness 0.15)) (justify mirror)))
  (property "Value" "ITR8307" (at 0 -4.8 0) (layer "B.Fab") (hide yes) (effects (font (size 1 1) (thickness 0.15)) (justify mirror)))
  (fp_line (start 1.85 1.8) (end 1.85 -1.8) (stroke (width 0.12) (type solid)) (layer "Edge.Cuts"))
  (fp_line (start 1.85 -1.8) (end -1.85 -1.8) (stroke (width 0.12) (type solid)) (layer "Edge.Cuts"))
  (fp_line (start -1.85 1.8) (end 1.85 1.8) (stroke (width 0.12) (type solid)) (layer "Edge.Cuts"))
  (fp_line (start -1.85 -1.8) (end -1.85 1.8) (stroke (width 0.12) (type solid)) (layer "Edge.Cuts"))
  (pad "1" smd roundrect (at -0.9 -2.8 180) (size 1.2 1.4) (layers "B.Cu" "B.Mask" "B.Paste") (roundrect_rratio 0.2) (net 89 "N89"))
  (pad "2" smd roundrect (at -0.9 2.8 180) (size 1.2 1.4) (layers "B.Cu" "B.Mask" "B.Paste") (roundrect_rratio 0.2) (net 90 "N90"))
  (pad "3" smd roundrect (at 0.9 -2.8 180) (size 1.2 1.4) (layers "B.Cu" "B.Mask" "B.Paste") (roundrect_rratio 0.2) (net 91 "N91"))
  (pad "4" smd roundrect (at 0.9 2.8 180) (size 1.2 1.4) (layers "B.Cu" "B.Mask" "B.Paste") (roundrect_rratio 0.2) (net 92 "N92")))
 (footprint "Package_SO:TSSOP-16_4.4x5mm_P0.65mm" (layer "B.Cu") (at 89.7125 79.2 180)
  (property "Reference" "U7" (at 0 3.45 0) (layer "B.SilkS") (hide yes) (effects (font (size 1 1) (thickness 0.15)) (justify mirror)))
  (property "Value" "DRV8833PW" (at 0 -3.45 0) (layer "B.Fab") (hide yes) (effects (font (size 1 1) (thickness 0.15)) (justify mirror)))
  (pad "1" smd roundrect (at -2.8625 2.275 180) (size 1.475 0.4) (layers "B.Cu" "B.Mask" "B.Paste") (roundrect_rratio 0.25) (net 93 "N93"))
  (pad "2" smd roundrect (at -2.8625 1.625 180) (size 1.475 0.4) (layers "B.Cu" "B.Mask" "B.Paste") (roundrect_rratio 0.25) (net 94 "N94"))
  (pad "3" smd roundrect (at -2.8625 0.975 180) (size 1.475 0.4) (layers "B.Cu" "B.Mask" "B.Paste") (roundrect_rratio 0.25) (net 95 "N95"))
  (pad "4" smd roundrect (at -2.8625 0.325 180) (size 1.475 0.4) (layers "B.Cu" "B.Mask" "B.Paste") (roundrect_rratio 0.25) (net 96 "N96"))
  (pad "5" smd roundrect (at -2.8625 -0.325 180) (size 1.475 0.4) (layers "B.Cu" "B.Mask" "B.Paste") (roundrect_rratio 0.25) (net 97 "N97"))
  (pad "6" smd roundrect (at -2.8625 -0.975 180) (size 1.475 0.4) (layers "B.Cu" "B.Mask" "B.Paste") (roundrect_rratio 0.25) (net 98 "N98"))
  (pad "7" smd roundrect (at -2.8625 -1.625 180) (size 1.475 0.4) (layers "B.Cu" "B.Mask" "B.Paste") (roundrect_rratio 0.25) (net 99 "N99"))
  (pad "8" smd roundrect (at -2.8625 -2.275 180) (size 1.475 0.4) (layers "B.Cu" "B.Mask" "B.Paste") (roundrect_rratio 0.25)
   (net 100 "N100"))
  (pad "9" smd roundrect (at 2.8625 -2.275 180) (size 1.475 0.4) (layers "B.Cu" "B.Mask" "B.Paste") (roundrect_rratio 0.25) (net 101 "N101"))
  (pad "10" smd roundrect (at 2.8625 -1.625 180) (size 1.475 0.4) (layers "B.Cu" "B.Mask" "B.Paste") (roundrect_rratio 0.25)
   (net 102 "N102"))
  (pad "11" smd roundrect (at 2.8625 -0.975 180) (size 1.475 0.4) (layers "B.Cu" "B.Mask" "B.Paste") (roundrect_rratio 0.25)
   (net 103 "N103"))
  (pad "12" smd roundrect (at 2.8625 -0.325 180) (size 1.475 0.4) (layers "B.Cu" "B.Mask" "B.Paste") (roundrect_rratio 0.25)
   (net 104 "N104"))
  (pad "13" smd roundrect (at 2.8625 0.325 180) (size 1.475 0.4) (layers "B.Cu" "B.Mask" "B.Paste") (roundrect_rratio 0.25) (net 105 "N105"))
  (pad "14" smd roundrect (at 2.8625 0.975 180) (size 1.475 0.4) (layers "B.Cu" "B.Mask" "B.Paste") (roundrect_rratio 0.25) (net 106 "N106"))
  (pad "15" smd roundrect (at 2.8625 1.625 180) (size 1.475 0.4) (layers "B.Cu" "B.Mask" "B.Paste") (roundrect_rratio 0.25) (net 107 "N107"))
  (pad "16" smd roundrect (at 2.8625 2.275 180) (size 1.475 0.4) (layers "B.Cu" "B.Mask" "B.Paste") (roundrect_rratio 0.25) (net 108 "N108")))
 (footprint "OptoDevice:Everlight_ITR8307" (layer "B.Cu") (at 77.45 53.55 180)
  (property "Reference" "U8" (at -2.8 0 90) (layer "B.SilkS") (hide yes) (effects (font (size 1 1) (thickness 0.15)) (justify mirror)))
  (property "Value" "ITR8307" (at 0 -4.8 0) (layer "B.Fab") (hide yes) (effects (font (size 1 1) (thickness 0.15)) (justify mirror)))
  (fp_line (start 1.85 1.8) (end 1.85 -1.8) (stroke (width 0.12) (type solid)) (layer "Edge.Cuts"))
  (fp_line (start 1.85 -1.8) (end -1.85 -1.8) (stroke (width 0.12) (type solid)) (layer "Edge.Cuts"))
  (fp_line (start -1.85 1.8) (end 1.85 1.8) (stroke (width 0.12) (type solid)) (layer "Edge.Cuts"))
  (fp_line (start -1.85 -1.8) (end -1.85 1.8) (stroke (width 0.12) (type solid)) (layer "Edge.Cuts"))
  (pad "1" smd roundrect (at -0.9 -2.8 180) (size 1.2 1.4) (layers "B.Cu" "B.Mask" "B.Paste") (roundrect_rratio 0.2) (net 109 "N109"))
  (pad "2" smd roundrect (at -0.9 2.8 180) (size 1.2 1.4) (layers "B.Cu" "B.Mask" "B.Paste") (roundrect_rratio 0.2) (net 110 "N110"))
  (pad "3" smd roundrect (at 0.9 -2.8 180) (size 1.2 1.4) (layers "B.Cu" "B.Mask" "B.Paste") (roundrect_rratio 0.2) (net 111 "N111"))
  (pad "4" smd roundrect (at 0.9 2.8 180) (size 1.2 1.4) (layers "B.Cu" "B.Mask" "B.Paste") (roundrect_rratio 0.2) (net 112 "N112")))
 (gr_line (start 103.7 98.7) (end 75.7 98.7) (stroke (width 0.05) (type default)) (layer "Edge.Cuts"))
 (gr_arc (start 74.7 49.7) (mid 74.992893 48.992893) (end 75.7 48.7) (stroke (width 0.05) (type default)) (layer "Edge.Cuts"))
 (gr_arc (start 103.7 48.7) (mid 104.407107 48.992893) (end 104.7 49.7) (stroke (width 0.05) (type default)) (layer "Edge.Cuts"))
 (gr_arc (start 75.7 98.7) (mid 74.992893 98.407107) (end 74.7 97.7) (stroke (width 0.05) (type default)) (layer "Edge.Cuts"))
 (gr_line (start 104.7 49.7) (end 104.7 97.7) (stroke (width 0.05) (type default)) (layer "Edge.Cuts"))
 (gr_arc (start 104.7 97.7) (mid 104.407107 98.407107) (end 103.7 98.7) (stroke (width 0.05) (type default)) (layer "Edge.Cuts"))
 (gr_line (start 75.7 48.7) (end 103.7 48.7) (stroke (width 0.05) (type default)) (layer "Edge.Cuts"))
 (gr_line (start 74.7 97.7) (end 74.7 49.7) (stroke (width 0.05) (type default)) (layer "Edge.Cuts"))
 (segment (start 88.15 64.2) (end 88.5 64.2) (width 0.3) (layer "F.Cu") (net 34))
 (segment (start 83.72 65.43) (end 84.55 64.6) (width 0.3) (layer "F.Cu") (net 34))
 (segment (start 80.95 65.43) (end 83.72 65.43) (width 0.3) (layer "F.Cu") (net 34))
 (segment (start 84.95 64.2) (end 88.15 64.2) (width 0.3) (layer "F.Cu") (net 34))
 (segment (start 84.55 64.6) (end 84.95 64.2) (width 0.3) (layer "F.Cu") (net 34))
 (segment (start 80.95 66.7) (end 84.55 66.7) (width 0.3) (layer "F.Cu") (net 33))
 (segment (start 84.55 66.7) (end 85.55 65.7) (width 0.3) (layer "F.Cu") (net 33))
 (segment (start 85.9 65.35) (end 86.85 65.35) (width 0.3) (layer "F.Cu") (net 33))
 (segment (start 85.55 65.7) (end 85.9 65.35) (width 0.3) (layer "F.Cu") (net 33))
 (segment (start 88.75 86.125) (end 88.75 84.41) (width 0.3) (layer "F.Cu") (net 32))
 (segment (start 90.65 86.125) (end 90.65 84.36) (width 0.3) (layer "F.Cu") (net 30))
 (segment (start 89.925 92.425) (end 89.925 91.1375) (width 0.2) (layer "F.Cu") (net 5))
 (segment (start 89.925 91.1375) (end 89.95 91.1125) (width 0.2) (layer "F.Cu") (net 5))
 (segment (start 89.8 92.55) (end 89.925 92.425) (width 0.2) (layer "F.Cu") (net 5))
 (segment (start 90.65 89.5) (end 90.65 88.4) (width 0.2) (layer "F.Cu") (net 5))
 (segment (start 89.95 91.1125) (end 89.95 90.2) (width 0.2) (layer "F.Cu") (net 5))
 (segment (start 88.95 91.1125) (end 88.95 92.4) (width 0.2) (layer "F.Cu") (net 5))
 (segment (start 89.1 92.55) (end 89.8 92.55) (width 0.2) (layer "F.Cu") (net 5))
 (segment (start 89.95 90.2) (end 90.65 89.5) (width 0.2) (layer "F.Cu") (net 5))
 (segment (start 88.95 92.4) (end 89.1 92.55) (width 0.2) (layer "F.Cu") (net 5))
 (segment (start 88.75 89.3) (end 89.45 90) (width 0.2) (layer "F.Cu") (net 4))
 (segment (start 89.45 90) (end 89.45 91.1125) (width 0.2) (layer "F.Cu") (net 4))
 (segment (start 88.75 88.4) (end 88.75 89.3) (width 0.2) (layer "F.Cu") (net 4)))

